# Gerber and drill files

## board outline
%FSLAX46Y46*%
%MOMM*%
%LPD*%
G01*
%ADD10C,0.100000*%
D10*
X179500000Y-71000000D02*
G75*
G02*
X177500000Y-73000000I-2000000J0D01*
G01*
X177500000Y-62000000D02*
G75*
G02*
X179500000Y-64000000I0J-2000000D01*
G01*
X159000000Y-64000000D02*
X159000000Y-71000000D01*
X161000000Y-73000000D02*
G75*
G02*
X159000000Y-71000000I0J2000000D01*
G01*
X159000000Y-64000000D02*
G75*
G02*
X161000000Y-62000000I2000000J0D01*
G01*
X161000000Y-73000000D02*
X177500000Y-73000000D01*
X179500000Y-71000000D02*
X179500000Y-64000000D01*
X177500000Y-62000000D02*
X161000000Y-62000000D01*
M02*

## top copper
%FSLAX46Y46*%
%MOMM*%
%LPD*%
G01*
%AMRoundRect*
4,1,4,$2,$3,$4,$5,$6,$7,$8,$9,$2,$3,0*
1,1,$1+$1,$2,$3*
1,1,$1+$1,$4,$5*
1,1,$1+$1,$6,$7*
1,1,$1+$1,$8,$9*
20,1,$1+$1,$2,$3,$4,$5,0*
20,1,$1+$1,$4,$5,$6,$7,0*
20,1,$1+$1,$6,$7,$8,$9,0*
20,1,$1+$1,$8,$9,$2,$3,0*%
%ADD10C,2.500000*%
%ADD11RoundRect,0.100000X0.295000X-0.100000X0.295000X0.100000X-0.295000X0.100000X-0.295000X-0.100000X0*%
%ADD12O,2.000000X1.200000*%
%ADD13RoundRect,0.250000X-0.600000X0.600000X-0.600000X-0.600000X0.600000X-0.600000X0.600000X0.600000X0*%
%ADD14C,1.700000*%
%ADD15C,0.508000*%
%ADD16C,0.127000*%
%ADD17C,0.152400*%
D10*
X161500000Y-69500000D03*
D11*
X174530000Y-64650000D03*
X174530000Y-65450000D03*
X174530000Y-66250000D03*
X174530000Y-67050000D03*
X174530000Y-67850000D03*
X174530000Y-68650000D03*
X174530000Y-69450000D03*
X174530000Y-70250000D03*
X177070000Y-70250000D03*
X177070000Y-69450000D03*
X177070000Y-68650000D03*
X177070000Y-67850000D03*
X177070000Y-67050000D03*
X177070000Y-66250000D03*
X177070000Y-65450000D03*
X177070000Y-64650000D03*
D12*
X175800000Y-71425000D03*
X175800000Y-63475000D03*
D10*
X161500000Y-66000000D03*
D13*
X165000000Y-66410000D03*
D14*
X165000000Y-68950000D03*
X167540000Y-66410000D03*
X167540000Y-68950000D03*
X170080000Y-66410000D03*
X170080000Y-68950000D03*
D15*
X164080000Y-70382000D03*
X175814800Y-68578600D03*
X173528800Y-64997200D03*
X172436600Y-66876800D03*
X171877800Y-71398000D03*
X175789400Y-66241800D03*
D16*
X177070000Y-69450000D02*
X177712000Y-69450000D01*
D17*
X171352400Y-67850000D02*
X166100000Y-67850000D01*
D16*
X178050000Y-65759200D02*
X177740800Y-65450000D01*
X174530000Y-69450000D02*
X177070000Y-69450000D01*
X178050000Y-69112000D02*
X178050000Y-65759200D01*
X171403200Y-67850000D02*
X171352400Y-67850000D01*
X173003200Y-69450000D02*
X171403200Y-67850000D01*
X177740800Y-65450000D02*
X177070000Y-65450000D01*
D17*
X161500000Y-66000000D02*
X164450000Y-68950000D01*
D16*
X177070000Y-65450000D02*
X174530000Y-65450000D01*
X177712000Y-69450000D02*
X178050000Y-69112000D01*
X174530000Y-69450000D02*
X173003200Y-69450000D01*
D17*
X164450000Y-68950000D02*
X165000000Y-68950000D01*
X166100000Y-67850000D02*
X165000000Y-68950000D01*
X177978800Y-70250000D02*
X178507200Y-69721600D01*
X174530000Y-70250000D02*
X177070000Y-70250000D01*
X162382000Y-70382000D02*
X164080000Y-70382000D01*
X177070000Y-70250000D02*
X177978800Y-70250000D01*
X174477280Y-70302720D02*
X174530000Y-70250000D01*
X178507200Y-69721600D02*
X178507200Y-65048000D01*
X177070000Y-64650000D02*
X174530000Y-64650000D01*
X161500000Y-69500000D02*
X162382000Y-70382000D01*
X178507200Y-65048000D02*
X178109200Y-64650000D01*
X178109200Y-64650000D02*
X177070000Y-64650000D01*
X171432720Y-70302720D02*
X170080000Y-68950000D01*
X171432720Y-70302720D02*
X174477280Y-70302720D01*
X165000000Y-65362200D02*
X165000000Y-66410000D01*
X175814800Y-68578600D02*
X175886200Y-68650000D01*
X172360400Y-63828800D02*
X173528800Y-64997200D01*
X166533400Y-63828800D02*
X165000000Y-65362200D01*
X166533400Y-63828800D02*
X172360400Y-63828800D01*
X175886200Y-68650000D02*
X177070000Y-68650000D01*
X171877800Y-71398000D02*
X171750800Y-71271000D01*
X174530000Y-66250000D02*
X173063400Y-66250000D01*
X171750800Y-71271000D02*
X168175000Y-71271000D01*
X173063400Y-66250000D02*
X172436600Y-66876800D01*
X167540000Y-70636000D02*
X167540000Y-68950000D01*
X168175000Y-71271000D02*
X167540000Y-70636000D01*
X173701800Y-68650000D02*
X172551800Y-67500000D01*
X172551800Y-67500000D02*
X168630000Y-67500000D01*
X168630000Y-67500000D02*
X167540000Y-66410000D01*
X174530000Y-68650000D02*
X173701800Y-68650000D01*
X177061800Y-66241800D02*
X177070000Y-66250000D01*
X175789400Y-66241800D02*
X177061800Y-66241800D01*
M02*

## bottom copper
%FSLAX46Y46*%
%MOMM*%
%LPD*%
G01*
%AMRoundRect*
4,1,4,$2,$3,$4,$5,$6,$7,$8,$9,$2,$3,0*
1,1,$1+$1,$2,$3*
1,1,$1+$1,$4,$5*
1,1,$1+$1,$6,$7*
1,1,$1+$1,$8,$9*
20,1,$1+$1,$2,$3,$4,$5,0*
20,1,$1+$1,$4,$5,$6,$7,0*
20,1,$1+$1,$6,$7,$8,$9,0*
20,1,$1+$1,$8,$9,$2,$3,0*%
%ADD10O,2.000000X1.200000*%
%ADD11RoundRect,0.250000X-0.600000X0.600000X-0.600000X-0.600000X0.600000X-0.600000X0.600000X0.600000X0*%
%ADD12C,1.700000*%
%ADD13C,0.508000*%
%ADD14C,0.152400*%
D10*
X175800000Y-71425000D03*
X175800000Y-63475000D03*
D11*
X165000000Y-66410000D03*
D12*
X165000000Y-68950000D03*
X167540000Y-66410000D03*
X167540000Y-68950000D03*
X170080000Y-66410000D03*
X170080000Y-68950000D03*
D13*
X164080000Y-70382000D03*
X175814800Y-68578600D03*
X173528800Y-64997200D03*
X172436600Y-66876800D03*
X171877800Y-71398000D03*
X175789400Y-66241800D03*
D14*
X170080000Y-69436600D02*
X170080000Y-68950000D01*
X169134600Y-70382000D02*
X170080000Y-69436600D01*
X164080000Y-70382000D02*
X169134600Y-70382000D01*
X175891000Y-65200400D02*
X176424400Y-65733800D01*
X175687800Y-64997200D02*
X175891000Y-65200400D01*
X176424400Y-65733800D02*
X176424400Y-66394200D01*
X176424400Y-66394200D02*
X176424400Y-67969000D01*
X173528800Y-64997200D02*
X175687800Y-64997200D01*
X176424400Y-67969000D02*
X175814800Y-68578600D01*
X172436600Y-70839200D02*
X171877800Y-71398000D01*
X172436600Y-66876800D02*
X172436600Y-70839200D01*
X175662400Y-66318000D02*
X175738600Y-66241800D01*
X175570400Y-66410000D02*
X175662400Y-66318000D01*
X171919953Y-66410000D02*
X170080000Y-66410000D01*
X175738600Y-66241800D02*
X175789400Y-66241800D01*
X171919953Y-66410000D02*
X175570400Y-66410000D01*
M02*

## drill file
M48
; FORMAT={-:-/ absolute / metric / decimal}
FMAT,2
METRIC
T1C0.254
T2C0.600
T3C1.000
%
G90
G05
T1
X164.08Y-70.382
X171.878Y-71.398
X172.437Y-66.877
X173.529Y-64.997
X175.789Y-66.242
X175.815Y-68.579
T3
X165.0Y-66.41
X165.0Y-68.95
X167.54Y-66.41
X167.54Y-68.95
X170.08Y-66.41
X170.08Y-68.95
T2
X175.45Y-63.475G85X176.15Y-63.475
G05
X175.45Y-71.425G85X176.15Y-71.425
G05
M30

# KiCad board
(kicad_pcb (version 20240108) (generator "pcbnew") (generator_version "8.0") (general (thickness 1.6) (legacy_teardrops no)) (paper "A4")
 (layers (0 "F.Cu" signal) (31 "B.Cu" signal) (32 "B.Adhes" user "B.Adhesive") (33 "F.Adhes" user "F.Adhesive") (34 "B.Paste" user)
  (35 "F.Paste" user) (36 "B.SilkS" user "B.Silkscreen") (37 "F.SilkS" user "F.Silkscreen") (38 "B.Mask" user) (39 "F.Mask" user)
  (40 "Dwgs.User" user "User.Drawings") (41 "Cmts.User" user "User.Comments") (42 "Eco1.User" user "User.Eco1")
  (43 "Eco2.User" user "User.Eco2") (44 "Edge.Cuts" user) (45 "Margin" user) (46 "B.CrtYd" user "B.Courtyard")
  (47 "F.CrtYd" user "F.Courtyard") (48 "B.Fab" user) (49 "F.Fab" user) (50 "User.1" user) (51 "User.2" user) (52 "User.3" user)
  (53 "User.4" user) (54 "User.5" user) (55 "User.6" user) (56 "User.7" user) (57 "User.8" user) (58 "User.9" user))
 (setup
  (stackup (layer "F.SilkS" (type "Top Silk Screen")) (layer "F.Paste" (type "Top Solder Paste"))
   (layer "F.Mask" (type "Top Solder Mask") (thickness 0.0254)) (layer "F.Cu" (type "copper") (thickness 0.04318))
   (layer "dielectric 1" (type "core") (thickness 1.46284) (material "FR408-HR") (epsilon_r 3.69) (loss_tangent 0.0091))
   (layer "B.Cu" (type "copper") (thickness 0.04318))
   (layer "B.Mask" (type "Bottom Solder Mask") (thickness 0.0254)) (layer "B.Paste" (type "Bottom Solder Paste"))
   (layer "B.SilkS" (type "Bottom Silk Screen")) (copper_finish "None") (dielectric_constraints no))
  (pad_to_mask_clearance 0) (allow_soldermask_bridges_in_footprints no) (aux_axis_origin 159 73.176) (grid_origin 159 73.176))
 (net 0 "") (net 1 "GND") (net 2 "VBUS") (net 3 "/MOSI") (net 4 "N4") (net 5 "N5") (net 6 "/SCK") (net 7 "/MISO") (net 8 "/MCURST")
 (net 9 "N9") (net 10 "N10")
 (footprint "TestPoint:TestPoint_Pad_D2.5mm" (layer "F.Cu") (at 161.5 69.5 -90)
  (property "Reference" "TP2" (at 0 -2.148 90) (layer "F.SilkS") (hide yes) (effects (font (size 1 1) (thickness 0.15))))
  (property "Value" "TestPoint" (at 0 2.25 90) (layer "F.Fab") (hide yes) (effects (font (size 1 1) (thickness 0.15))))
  (pad "1" smd circle (at 0 0 270) (size 2.5 2.5) (layers "F.Cu" "F.Mask") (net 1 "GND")))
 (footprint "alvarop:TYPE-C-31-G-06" (layer "F.Cu") (at 175.8 67.45 90)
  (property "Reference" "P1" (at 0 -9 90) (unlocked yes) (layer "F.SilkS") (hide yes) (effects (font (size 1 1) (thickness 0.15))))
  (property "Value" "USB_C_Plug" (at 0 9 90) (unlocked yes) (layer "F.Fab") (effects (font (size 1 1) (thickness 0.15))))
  (pad "A1" smd roundrect (at 2.8 -1.27 90) (size 0.4 0.79) (layers "F.Cu" "F.Paste" "F.Mask") (roundrect_rratio 0.25) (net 1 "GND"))
  (pad "A4" smd roundrect (at 2 -1.27 90) (size 0.4 0.79) (layers "F.Cu" "F.Paste" "F.Mask") (roundrect_rratio 0.25) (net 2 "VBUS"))
  (pad "A5" smd roundrect (at 1.2 -1.27 90) (size 0.4 0.79) (layers "F.Cu" "F.Paste" "F.Mask") (roundrect_rratio 0.25) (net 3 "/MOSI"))
  (pad "A6" smd roundrect (at 0.4 -1.27 90) (size 0.4 0.79) (layers "F.Cu" "F.Paste" "F.Mask") (roundrect_rratio 0.25) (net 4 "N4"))
  (pad "A7" smd roundrect (at -0.4 -1.27 90) (size 0.4 0.79) (layers "F.Cu" "F.Paste" "F.Mask") (roundrect_rratio 0.25) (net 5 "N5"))
  (pad "A8" smd roundrect (at -1.2 -1.27 90) (size 0.4 0.79) (layers "F.Cu" "F.Paste" "F.Mask") (roundrect_rratio 0.25) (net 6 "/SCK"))
  (pad "A9" smd roundrect (at -2 -1.27 90) (size 0.4 0.79) (layers "F.Cu" "F.Paste" "F.Mask") (roundrect_rratio 0.25) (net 2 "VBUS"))
  (pad "A12" smd roundrect (at -2.8 -1.27 90) (size 0.4 0.79) (layers "F.Cu" "F.Paste" "F.Mask") (roundrect_rratio 0.25) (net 1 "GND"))
  (pad "B1" smd roundrect (at -2.8 1.27 90) (size 0.4 0.79) (layers "F.Cu" "F.Paste" "F.Mask") (roundrect_rratio 0.25) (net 1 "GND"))
  (pad "B4" smd roundrect (at -2 1.27 90) (size 0.4 0.79) (layers "F.Cu" "F.Paste" "F.Mask") (roundrect_rratio 0.25) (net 2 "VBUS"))
  (pad "B5" smd roundrect (at -1.2 1.27 90) (size 0.4 0.79) (layers "F.Cu" "F.Paste" "F.Mask") (roundrect_rratio 0.25) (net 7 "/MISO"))
  (pad "B6" smd roundrect (at -0.4 1.27 90) (size 0.4 0.79) (layers "F.Cu" "F.Paste" "F.Mask") (roundrect_rratio 0.25))
  (pad "B7" smd roundrect (at 0.4 1.27 90) (size 0.4 0.79) (layers "F.Cu" "F.Paste" "F.Mask") (roundrect_rratio 0.25))
  (pad "B8" smd roundrect (at 1.2 1.27 90) (size 0.4 0.79) (layers "F.Cu" "F.Paste" "F.Mask") (roundrect_rratio 0.25) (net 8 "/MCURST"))
  (pad "B9" smd roundrect (at 2 1.27 90) (size 0.4 0.79) (layers "F.Cu" "F.Paste" "F.Mask") (roundrect_rratio 0.25) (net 2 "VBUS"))
  (pad "B12" smd roundrect (at 2.8 1.27 90) (size 0.4 0.79) (layers "F.Cu" "F.Paste" "F.Mask") (roundrect_rratio 0.25) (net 1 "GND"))
  (pad "S1" thru_hole oval (at -3.975 0 90) (size 1.2 2) (drill oval 0.6 1.3) (layers "*.Cu" "*.Mask") (remove_unused_layers no)
   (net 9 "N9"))
  (pad "S1" thru_hole oval (at 3.975 0 90) (size 1.2 2) (drill oval 0.6 1.3) (layers "*.Cu" "*.Mask") (remove_unused_layers no)
   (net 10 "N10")))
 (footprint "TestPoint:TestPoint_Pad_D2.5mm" (layer "F.Cu") (at 161.5 66 -90)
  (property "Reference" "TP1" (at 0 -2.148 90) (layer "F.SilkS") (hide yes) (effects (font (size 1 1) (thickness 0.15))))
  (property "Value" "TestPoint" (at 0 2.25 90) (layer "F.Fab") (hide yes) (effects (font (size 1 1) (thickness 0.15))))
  (pad "1" smd circle (at 0 0 270) (size 2.5 2.5) (layers "F.Cu" "F.Mask") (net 2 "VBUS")))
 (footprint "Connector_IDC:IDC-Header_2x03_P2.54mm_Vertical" (layer "B.Cu") (at 165 66.41 -90)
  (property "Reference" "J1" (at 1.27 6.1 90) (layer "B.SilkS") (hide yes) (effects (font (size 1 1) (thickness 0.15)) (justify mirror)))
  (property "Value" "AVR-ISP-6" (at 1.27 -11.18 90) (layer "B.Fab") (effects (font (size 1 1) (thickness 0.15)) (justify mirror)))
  (pad "1" thru_hole roundrect (at 0 0 270) (size 1.7 1.7) (drill 1) (layers "*.Cu" "*.Mask") (remove_unused_layers no)
   (roundrect_rratio 0.1470588235) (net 7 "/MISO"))
  (pad "2" thru_hole circle (at 2.54 0 270) (size 1.7 1.7) (drill 1) (layers "*.Cu" "*.Mask") (remove_unused_layers no) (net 2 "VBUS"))
  (pad "3" thru_hole circle (at 0 -2.54 270) (size 1.7 1.7) (drill 1) (layers "*.Cu" "*.Mask") (remove_unused_layers no) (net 6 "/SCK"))
  (pad "4" thru_hole circle (at 2.54 -2.54 270) (size 1.7 1.7) (drill 1) (layers "*.Cu" "*.Mask") (remove_unused_layers no) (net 3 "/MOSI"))
  (pad "5" thru_hole circle (at 0 -5.08 270) (size 1.7 1.7) (drill 1) (layers "*.Cu" "*.Mask") (remove_unused_layers no) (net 8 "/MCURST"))
  (pad "6" thru_hole circle (at 2.54 -5.08 270) (size 1.7 1.7) (drill 1) (layers "*.Cu" "*.Mask") (remove_unused_layers no) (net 1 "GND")))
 (gr_arc (start 179.5 71) (mid 178.914214 72.414214) (end 177.5 73) (stroke (width 0.1) (type solid)) (layer "Edge.Cuts"))
 (gr_arc (start 177.5 62) (mid 178.914214 62.585786) (end 179.5 64) (stroke (width 0.1) (type solid)) (layer "Edge.Cuts"))
 (gr_line (start 159 64) (end 159 71) (stroke (width 0.1) (type solid)) (layer "Edge.Cuts"))
 (gr_arc (start 161 73) (mid 159.585786 72.414214) (end 159 71) (stroke (width 0.1) (type solid)) (layer "Edge.Cuts"))
 (gr_arc (start 159 64) (mid 159.585786 62.585786) (end 161 62) (stroke (width 0.1) (type solid)) (layer "Edge.Cuts"))
 (gr_line (start 161 73) (end 177.5 73) (stroke (width 0.1) (type solid)) (layer "Edge.Cuts"))
 (gr_line (start 179.5 71) (end 179.5 64) (stroke (width 0.1) (type solid)) (layer "Edge.Cuts"))
 (gr_line (start 177.5 62) (end 161 62) (stroke (width 0.1) (type solid)) (layer "Edge.Cuts"))
 (segment (start 177.07 69.45) (end 177.712 69.45) (width 0.127) (layer "F.Cu") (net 2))
 (segment (start 171.3524 67.85) (end 166.1 67.85) (width 0.1524) (layer "F.Cu") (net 2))
 (segment (start 178.05 65.7592) (end 177.7408 65.45) (width 0.127) (layer "F.Cu") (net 2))
 (segment (start 174.53 69.45) (end 177.07 69.45) (width 0.127) (layer "F.Cu") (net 2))
 (segment (start 178.05 69.112) (end 178.05 65.7592) (width 0.127) (layer "F.Cu") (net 2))
 (segment (start 171.4032 67.85) (end 171.3524 67.85) (width 0.127) (layer "F.Cu") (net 2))
 (segment (start 173.0032 69.45) (end 171.4032 67.85) (width 0.127) (layer "F.Cu") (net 2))
 (segment (start 177.7408 65.45) (end 177.07 65.45) (width 0.127) (layer "F.Cu") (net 2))
 (segment (start 161.5 66) (end 164.45 68.95) (width 0.1524) (layer "F.Cu") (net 2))
 (segment (start 177.07 65.45) (end 174.53 65.45) (width 0.127) (layer "F.Cu") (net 2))
 (segment (start 177.712 69.45) (end 178.05 69.112) (width 0.127) (layer "F.Cu") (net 2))
 (segment (start 174.53 69.45) (end 173.0032 69.45) (width 0.127) (layer "F.Cu") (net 2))
 (segment (start 164.45 68.95) (end 165 68.95) (width 0.1524) (layer "F.Cu") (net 2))
 (segment (start 166.1 67.85) (end 165 68.95) (width 0.1524) (layer "F.Cu") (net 2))
 (segment (start 177.9788 70.25) (end 178.5072 69.7216) (width 0.1524) (layer "F.Cu") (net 1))
 (segment (start 174.53 70.25) (end 177.07 70.25) (width 0.1524) (layer "F.Cu") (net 1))
 (segment (start 162.382 70.382) (end 164.08 70.382) (width 0.1524) (layer "F.Cu") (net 1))
 (segment (start 177.07 70.25) (end 177.9788 70.25) (width 0.1524) (layer "F.Cu") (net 1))
 (segment (start 174.47728 70.30272) (end 174.53 70.25) (width 0.1524) (layer "F.Cu") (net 1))
 (segment (start 178.5072 69.7216) (end 178.5072 65.048) (width 0.1524) (layer "F.Cu") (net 1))
 (segment (start 177.07 64.65) (end 174.53 64.65) (width 0.1524) (layer "F.Cu") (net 1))
 (segment (start 161.5 69.5) (end 162.382 70.382) (width 0.1524) (layer "F.Cu") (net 1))
 (segment (start 178.5072 65.048) (end 178.1092 64.65) (width 0.1524) (layer "F.Cu") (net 1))
 (segment (start 178.1092 64.65) (end 177.07 64.65) (width 0.1524) (layer "F.Cu") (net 1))
 (segment (start 171.43272 70.30272) (end 170.08 68.95) (width 0.1524) (layer "F.Cu") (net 1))
 (segment (start 171.43272 70.30272) (end 174.47728 70.30272) (width 0.1524) (layer "F.Cu") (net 1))
 (via (at 164.08 70.382) (size 0.508) (drill 0.254) (layers "F.Cu" "B.Cu") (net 1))
 (segment (start 170.08 69.4366) (end 170.08 68.95) (width 0.1524) (layer "B.Cu") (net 1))
 (segment (start 169.1346 70.382) (end 170.08 69.4366) (width 0.1524) (layer "B.Cu") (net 1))
 (segment (start 164.08 70.382) (end 169.1346 70.382) (width 0.1524) (layer "B.Cu") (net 1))
 (segment (start 165 65.3622) (end 165 66.41) (width 0.1524) (layer "F.Cu") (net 7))
 (segment (start 175.8148 68.5786) (end 175.8862 68.65) (width 0.1524) (layer "F.Cu") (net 7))
 (segment (start 172.3604 63.8288) (end 173.5288 64.9972) (width 0.1524) (layer "F.Cu") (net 7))
 (segment (start 166.5334 63.8288) (end 165 65.3622) (width 0.1524) (layer "F.Cu") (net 7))
 (segment (start 166.5334 63.8288) (end 172.3604 63.8288) (width 0.1524) (layer "F.Cu") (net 7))
 (segment (start 175.8862 68.65) (end 177.07 68.65) (width 0.1524) (layer "F.Cu") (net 7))
 (via (at 175.8148 68.5786) (size 0.508) (drill 0.254) (layers "F.Cu" "B.Cu") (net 7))
 (via (at 173.5288 64.9972) (size 0.508) (drill 0.254) (layers "F.Cu" "B.Cu") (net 7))
 (segment (start 175.891 65.2004) (end 176.4244 65.7338) (width 0.1524) (layer "B.Cu") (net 7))
 (segment (start 175.6878 64.9972) (end 175.891 65.2004) (width 0.1524) (layer "B.Cu") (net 7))
 (segment (start 176.4244 65.7338) (end 176.4244 66.3942) (width 0.1524) (layer "B.Cu") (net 7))
 (segment (start 176.4244 66.3942) (end 176.4244 67.969) (width 0.1524) (layer "B.Cu") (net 7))
 (segment (start 173.5288 64.9972) (end 175.6878 64.9972) (width 0.1524) (layer "B.Cu") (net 7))
 (segment (start 176.4244 67.969) (end 175.8148 68.5786) (width 0.1524) (layer "B.Cu") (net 7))
 (segment (start 171.8778 71.398) (end 171.7508 71.271) (width 0.1524) (layer "F.Cu") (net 3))
 (segment (start 174.53 66.25) (end 173.0634 66.25) (width 0.1524) (layer "F.Cu") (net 3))
 (segment (start 171.7508 71.271) (end 168.175 71.271) (width 0.1524) (layer "F.Cu") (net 3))
 (segment (start 173.0634 66.25) (end 172.4366 66.8768) (width 0.1524) (layer "F.Cu") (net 3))
 (segment (start 167.54 70.636) (end 167.54 68.95) (width 0.1524) (layer "F.Cu") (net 3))
 (segment (start 168.175 71.271) (end 167.54 70.636) (width 0.1524) (layer "F.Cu") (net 3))
 (via (at 172.4366 66.8768) (size 0.508) (drill 0.254) (layers "F.Cu" "B.Cu") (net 3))
 (via (at 171.8778 71.398) (size 0.508) (drill 0.254) (layers "F.Cu" "B.Cu") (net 3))
 (segment (start 172.4366 70.8392) (end 171.8778 71.398) (width 0.1524) (layer "B.Cu") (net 3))
 (segment (start 172.4366 66.8768) (end 172.4366 70.8392) (width 0.1524) (layer "B.Cu") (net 3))
 (segment (start 173.7018 68.65) (end 172.5518 67.5) (width 0.1524) (layer "F.Cu") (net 6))
 (segment (start 172.5518 67.5) (end 168.63 67.5) (width 0.1524) (layer "F.Cu") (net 6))
 (segment (start 168.63 67.5) (end 167.54 66.41) (width 0.1524) (layer "F.Cu") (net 6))
 (segment (start 174.53 68.65) (end 173.7018 68.65) (width 0.1524) (layer "F.Cu") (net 6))
 (segment (start 177.0618 66.2418) (end 177.07 66.25) (width 0.1524) (layer "F.Cu") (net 8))
 (segment (start 175.7894 66.2418) (end 177.0618 66.2418) (width 0.1524) (layer "F.Cu") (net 8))
 (via (at 175.7894 66.2418) (size 0.508) (drill 0.254) (layers "F.Cu" "B.Cu") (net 8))
 (segment (start 175.6624 66.318) (end 175.7386 66.2418) (width 0.1524) (layer "B.Cu") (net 8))
 (segment (start 175.5704 66.41) (end 175.6624 66.318) (width 0.1524) (layer "B.Cu") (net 8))
 (segment (start 171.919953 66.41) (end 170.08 66.41) (width 0.1524) (layer "B.Cu") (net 8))
 (segment (start 175.7386 66.2418) (end 175.7894 66.2418) (width 0.1524) (layer "B.Cu") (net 8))
 (segment (start 171.919953 66.41) (end 175.5704 66.41) (width 0.1524) (layer "B.Cu") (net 8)))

